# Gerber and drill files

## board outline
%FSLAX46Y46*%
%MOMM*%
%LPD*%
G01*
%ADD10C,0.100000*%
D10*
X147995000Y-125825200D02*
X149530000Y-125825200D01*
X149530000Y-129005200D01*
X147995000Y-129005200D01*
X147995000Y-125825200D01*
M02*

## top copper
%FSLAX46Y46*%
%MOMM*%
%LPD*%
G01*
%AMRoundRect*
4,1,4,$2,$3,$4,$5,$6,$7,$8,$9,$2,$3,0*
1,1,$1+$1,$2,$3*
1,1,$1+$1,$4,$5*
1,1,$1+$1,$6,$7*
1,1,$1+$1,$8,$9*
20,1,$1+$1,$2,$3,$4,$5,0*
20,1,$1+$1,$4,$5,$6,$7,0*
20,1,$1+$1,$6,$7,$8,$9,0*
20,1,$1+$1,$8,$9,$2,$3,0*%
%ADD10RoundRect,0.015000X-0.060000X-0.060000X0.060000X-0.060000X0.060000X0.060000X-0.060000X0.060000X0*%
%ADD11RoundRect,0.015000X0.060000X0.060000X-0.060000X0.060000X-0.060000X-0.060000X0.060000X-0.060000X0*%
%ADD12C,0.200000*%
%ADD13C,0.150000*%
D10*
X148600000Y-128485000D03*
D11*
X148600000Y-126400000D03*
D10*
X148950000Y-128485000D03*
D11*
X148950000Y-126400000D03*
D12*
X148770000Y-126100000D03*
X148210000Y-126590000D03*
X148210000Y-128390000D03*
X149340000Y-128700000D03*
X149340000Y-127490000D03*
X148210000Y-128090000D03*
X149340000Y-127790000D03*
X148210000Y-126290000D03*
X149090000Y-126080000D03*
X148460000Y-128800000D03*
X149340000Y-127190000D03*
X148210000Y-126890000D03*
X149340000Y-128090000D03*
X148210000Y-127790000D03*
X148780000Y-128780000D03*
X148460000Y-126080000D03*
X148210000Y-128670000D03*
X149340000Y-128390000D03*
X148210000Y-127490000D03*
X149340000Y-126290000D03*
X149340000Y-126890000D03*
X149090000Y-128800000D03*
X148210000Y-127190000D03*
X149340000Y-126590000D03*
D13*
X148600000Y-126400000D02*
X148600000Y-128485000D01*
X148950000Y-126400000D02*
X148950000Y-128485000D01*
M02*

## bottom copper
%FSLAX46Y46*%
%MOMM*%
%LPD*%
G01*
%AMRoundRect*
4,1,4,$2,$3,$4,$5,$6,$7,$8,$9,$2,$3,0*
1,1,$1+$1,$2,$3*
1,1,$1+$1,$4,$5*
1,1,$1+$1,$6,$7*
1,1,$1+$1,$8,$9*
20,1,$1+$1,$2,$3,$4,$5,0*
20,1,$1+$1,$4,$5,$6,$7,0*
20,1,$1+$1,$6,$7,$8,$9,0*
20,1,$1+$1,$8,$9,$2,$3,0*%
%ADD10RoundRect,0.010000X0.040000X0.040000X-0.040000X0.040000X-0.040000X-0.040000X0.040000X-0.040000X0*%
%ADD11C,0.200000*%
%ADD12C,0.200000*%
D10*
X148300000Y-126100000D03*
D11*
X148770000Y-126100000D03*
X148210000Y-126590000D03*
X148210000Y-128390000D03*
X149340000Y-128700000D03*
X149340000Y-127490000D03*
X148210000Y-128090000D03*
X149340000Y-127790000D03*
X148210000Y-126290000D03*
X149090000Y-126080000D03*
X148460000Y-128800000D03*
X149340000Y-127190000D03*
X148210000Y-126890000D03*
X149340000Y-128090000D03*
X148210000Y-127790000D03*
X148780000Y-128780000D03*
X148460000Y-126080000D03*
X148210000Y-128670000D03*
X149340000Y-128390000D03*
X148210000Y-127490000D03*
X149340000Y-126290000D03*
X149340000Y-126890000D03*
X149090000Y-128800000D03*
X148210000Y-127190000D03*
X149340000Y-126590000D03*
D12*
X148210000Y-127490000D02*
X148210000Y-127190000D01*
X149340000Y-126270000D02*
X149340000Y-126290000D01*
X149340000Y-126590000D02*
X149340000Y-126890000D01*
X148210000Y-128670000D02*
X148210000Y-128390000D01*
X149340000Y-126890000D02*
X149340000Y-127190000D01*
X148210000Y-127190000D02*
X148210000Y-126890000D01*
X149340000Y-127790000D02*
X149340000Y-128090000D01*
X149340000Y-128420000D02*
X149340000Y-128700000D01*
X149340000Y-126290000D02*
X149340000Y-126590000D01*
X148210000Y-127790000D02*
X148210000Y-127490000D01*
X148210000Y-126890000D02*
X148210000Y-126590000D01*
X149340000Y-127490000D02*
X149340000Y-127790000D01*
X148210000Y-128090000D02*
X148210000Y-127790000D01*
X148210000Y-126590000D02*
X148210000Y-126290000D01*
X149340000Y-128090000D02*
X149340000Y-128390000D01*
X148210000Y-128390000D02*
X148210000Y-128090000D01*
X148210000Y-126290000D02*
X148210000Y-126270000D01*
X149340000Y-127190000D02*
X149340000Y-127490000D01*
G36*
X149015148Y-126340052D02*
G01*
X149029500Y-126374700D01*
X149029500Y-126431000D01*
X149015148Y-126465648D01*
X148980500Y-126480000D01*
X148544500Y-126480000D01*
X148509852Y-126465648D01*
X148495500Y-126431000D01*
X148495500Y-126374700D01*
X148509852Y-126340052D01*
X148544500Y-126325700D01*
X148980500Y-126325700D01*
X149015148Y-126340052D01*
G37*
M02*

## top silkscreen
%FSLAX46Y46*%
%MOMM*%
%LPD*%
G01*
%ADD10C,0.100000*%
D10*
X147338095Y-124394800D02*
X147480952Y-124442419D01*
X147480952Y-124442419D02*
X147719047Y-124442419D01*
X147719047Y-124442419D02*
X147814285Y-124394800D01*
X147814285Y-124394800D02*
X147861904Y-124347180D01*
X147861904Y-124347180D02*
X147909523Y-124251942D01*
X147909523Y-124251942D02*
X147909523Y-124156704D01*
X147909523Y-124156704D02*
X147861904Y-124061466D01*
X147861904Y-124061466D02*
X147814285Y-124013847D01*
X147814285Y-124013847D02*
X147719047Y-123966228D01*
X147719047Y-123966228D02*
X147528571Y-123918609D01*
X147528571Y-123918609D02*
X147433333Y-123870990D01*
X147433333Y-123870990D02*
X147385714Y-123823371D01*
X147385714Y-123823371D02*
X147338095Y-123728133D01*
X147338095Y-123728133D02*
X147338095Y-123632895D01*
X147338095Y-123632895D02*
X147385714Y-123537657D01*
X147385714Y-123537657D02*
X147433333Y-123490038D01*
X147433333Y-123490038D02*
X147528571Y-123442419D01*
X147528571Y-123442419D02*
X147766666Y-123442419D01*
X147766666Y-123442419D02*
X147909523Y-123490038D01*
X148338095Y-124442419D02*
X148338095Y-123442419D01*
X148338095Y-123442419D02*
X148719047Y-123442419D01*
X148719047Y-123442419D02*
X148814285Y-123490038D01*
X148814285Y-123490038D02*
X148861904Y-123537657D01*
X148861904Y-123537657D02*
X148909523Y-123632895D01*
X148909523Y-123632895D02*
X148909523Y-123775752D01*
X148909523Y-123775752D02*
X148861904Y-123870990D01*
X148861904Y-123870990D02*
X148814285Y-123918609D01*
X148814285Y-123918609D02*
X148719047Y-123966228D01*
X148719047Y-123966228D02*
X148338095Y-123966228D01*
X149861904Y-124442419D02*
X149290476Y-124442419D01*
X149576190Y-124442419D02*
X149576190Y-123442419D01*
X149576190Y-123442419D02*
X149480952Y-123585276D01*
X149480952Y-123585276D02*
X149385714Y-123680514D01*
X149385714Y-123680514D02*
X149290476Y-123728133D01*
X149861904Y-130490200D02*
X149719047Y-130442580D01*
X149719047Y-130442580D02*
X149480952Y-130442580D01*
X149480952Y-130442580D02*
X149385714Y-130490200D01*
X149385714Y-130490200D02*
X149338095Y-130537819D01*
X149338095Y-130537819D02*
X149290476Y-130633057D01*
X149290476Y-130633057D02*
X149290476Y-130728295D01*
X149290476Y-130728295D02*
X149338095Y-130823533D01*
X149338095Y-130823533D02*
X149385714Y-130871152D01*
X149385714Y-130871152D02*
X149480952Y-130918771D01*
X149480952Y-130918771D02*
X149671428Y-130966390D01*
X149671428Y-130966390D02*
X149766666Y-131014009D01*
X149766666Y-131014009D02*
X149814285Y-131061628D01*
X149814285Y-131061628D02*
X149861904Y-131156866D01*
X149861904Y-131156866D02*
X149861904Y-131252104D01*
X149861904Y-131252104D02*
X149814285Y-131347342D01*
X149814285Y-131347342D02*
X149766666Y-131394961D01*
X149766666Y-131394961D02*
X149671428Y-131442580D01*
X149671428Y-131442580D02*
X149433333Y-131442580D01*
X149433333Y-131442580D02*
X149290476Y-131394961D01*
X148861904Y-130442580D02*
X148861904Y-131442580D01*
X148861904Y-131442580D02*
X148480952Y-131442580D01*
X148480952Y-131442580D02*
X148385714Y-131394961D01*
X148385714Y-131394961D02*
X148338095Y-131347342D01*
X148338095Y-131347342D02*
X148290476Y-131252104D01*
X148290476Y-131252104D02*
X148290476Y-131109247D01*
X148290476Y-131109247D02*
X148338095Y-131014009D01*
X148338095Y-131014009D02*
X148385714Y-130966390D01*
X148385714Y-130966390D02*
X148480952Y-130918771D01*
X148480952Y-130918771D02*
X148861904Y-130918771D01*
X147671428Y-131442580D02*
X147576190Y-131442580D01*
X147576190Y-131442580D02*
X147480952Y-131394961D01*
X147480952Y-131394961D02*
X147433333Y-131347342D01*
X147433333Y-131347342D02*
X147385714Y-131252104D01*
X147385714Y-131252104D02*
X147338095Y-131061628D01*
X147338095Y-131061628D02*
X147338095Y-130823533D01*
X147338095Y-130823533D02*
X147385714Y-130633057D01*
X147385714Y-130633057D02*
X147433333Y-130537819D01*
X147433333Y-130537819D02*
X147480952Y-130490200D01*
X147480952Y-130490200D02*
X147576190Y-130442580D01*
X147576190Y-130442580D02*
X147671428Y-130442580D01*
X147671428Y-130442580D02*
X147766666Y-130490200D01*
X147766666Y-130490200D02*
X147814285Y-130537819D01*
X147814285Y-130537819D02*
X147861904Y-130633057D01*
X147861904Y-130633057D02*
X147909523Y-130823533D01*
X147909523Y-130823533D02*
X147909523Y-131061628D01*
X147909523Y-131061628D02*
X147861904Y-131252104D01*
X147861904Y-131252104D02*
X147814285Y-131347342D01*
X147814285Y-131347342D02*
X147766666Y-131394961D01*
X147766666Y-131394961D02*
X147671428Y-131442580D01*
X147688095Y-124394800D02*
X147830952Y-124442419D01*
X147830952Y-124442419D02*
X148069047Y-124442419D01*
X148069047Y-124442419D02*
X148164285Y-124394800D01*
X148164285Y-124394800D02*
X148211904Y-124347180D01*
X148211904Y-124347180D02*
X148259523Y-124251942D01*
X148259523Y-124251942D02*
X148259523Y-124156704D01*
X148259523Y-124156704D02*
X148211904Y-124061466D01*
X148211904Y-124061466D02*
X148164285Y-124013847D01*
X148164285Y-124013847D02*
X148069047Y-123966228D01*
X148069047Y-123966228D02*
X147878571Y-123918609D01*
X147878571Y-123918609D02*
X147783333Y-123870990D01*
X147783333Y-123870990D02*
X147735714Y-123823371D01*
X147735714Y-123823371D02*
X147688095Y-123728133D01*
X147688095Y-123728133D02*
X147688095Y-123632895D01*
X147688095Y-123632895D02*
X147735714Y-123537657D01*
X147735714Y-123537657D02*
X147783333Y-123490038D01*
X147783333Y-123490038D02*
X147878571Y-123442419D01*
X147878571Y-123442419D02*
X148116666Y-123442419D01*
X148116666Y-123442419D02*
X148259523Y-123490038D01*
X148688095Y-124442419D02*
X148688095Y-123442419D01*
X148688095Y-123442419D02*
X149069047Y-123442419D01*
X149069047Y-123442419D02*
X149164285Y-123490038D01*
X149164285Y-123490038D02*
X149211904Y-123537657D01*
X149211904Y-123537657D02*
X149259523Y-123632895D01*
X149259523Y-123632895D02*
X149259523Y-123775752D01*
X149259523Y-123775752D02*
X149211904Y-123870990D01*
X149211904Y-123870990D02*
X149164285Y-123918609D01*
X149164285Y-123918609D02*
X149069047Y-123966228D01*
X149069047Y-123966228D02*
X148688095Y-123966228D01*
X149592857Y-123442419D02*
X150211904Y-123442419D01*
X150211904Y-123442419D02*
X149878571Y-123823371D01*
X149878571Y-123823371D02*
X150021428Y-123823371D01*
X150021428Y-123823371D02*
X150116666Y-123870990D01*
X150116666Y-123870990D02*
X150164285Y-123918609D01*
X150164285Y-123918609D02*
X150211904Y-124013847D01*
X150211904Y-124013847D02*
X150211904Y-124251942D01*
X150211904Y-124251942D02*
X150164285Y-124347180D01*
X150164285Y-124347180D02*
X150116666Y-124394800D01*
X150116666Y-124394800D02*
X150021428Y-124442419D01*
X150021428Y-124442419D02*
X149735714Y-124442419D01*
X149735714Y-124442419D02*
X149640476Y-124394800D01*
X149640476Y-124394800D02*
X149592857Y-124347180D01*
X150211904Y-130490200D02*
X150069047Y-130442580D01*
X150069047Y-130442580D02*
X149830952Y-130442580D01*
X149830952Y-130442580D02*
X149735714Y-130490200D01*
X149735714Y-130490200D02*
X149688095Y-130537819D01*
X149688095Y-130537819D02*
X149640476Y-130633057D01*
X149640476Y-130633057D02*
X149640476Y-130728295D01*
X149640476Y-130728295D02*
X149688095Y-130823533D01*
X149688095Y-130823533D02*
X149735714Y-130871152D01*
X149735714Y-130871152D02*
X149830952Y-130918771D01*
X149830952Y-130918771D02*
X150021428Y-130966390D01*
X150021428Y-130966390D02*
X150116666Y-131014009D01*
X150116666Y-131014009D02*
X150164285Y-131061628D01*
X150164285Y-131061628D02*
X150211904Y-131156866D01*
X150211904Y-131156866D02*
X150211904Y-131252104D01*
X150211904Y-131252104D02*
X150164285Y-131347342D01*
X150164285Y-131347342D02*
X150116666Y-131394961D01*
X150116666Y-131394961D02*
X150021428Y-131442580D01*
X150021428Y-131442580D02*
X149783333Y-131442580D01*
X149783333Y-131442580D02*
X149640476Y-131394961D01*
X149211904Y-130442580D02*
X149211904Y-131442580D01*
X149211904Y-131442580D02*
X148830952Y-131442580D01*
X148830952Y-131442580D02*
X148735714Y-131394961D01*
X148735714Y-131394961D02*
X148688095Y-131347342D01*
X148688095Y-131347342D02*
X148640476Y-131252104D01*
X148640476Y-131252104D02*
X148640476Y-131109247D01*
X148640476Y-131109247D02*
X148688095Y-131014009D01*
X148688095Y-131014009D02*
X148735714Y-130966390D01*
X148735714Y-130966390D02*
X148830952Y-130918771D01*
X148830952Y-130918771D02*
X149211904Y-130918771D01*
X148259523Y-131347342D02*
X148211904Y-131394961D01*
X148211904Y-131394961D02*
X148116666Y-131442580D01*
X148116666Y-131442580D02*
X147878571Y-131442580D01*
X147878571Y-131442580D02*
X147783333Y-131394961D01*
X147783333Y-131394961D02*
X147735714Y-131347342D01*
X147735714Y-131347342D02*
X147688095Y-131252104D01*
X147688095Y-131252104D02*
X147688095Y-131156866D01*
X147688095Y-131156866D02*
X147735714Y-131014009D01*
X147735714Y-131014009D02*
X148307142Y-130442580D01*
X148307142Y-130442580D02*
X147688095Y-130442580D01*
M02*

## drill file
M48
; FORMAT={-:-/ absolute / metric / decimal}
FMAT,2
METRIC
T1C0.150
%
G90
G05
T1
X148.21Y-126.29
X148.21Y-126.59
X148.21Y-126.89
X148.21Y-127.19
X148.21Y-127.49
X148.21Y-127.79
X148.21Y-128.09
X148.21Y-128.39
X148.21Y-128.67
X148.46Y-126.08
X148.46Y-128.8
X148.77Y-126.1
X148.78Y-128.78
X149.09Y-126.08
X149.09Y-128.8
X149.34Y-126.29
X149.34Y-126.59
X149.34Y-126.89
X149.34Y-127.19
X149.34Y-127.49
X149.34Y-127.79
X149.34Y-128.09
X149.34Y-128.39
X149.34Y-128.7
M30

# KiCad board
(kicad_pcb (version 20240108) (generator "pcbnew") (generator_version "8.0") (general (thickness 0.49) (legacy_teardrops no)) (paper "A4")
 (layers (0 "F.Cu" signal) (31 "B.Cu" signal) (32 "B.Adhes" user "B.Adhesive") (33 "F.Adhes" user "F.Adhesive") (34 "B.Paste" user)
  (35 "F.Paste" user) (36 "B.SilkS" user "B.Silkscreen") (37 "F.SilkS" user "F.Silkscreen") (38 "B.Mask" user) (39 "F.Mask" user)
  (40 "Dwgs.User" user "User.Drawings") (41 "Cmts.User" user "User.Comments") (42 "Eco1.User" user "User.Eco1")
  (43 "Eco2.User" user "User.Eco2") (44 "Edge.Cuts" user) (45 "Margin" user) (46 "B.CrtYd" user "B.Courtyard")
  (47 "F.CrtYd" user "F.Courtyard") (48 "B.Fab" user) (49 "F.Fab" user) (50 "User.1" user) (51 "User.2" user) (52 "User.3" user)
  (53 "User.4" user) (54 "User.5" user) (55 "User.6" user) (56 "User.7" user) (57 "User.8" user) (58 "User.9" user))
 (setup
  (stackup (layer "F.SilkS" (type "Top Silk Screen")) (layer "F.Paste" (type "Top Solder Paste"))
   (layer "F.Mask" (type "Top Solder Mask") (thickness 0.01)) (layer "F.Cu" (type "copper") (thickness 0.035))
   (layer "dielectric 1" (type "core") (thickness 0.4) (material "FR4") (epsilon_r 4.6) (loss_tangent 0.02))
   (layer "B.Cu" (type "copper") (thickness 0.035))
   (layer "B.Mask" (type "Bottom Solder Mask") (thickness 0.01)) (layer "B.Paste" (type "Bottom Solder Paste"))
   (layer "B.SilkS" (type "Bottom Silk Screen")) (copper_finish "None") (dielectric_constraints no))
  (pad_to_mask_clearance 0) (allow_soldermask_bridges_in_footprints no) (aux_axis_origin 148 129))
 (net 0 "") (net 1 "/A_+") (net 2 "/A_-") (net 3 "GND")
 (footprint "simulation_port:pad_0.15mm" (layer "F.Cu") (at 148.6 128.485)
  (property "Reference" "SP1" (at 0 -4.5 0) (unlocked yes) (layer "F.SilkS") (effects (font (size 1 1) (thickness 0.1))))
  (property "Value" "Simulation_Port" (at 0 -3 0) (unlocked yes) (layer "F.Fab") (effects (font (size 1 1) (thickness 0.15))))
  (pad "1" smd roundrect (at 0 0) (size 0.15 0.15) (layers "F.Cu" "F.Paste" "F.Mask") (roundrect_rratio 0.1) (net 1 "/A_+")
   (thermal_bridge_angle 45)
   (teardrops (best_length_ratio 0.5) (max_length 1) (best_width_ratio 1) (max_width 2) (curve_points 0) (filter_ratio 0.9) (enabled yes)
    (allow_two_segments yes) (prefer_zone_connections yes))))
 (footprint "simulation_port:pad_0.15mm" (layer "F.Cu") (at 148.6 126.4 180)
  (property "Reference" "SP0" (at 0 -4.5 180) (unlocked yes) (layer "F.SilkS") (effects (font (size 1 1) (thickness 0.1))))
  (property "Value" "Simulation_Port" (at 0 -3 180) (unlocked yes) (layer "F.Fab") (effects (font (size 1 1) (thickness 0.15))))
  (pad "1" smd roundrect (at 0 0 180) (size 0.15 0.15) (layers "F.Cu" "F.Paste" "F.Mask") (roundrect_rratio 0.1) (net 1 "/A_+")
   (thermal_bridge_angle 45)
   (teardrops (best_length_ratio 0.5) (max_length 1) (best_width_ratio 1) (max_width 2) (curve_points 0) (filter_ratio 0.9) (enabled yes)
    (allow_two_segments yes) (prefer_zone_connections yes))))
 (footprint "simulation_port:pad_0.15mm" (layer "F.Cu") (at 148.95 128.485)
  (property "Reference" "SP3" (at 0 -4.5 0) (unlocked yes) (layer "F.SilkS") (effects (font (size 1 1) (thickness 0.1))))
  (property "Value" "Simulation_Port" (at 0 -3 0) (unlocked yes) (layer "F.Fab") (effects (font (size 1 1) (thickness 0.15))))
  (pad "1" smd roundrect (at 0 0) (size 0.15 0.15) (layers "F.Cu" "F.Paste" "F.Mask") (roundrect_rratio 0.1) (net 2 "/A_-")
   (thermal_bridge_angle 45)
   (teardrops (best_length_ratio 0.5) (max_length 1) (best_width_ratio 1) (max_width 2) (curve_points 0) (filter_ratio 0.9) (enabled yes)
    (allow_two_segments yes) (prefer_zone_connections yes))))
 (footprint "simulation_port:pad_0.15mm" (layer "F.Cu") (at 148.95 126.4 180)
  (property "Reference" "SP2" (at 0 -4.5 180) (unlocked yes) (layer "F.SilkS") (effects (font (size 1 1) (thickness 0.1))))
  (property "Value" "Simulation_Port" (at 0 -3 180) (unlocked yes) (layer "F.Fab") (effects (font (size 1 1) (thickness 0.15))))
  (pad "1" smd roundrect (at 0 0 180) (size 0.15 0.15) (layers "F.Cu" "F.Paste" "F.Mask") (roundrect_rratio 0.1) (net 2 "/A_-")
   (thermal_bridge_angle 45)
   (teardrops (best_length_ratio 0.5) (max_length 1) (best_width_ratio 1) (max_width 2) (curve_points 0) (filter_ratio 0.9) (enabled yes)
    (allow_two_segments yes) (prefer_zone_connections yes))))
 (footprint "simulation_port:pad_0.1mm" (layer "B.Cu") (at 148.3 126.1 180)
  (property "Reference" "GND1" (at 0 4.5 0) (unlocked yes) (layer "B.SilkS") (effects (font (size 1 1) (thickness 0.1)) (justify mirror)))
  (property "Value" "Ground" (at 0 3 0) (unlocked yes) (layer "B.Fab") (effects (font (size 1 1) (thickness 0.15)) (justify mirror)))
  (pad "1" smd roundrect (at 0 0 180) (size 0.1 0.1) (layers "B.Cu" "B.Paste" "B.Mask") (roundrect_rratio 0.1) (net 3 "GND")
   (thermal_bridge_angle 45)
   (teardrops (best_length_ratio 0.5) (max_length 1) (best_width_ratio 1) (max_width 2) (curve_points 0) (filter_ratio 0.9) (enabled yes)
    (allow_two_segments yes) (prefer_zone_connections yes))))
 (gr_rect (start 147.995 125.8252) (end 149.53 129.0052) (stroke (width 0.1) (type solid)) (fill none) (layer "Edge.Cuts"))
 (via (at 148.77 126.1) (size 0.2) (drill 0.15) (layers "F.Cu" "B.Cu") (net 3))
 (via (at 148.21 126.59) (size 0.2) (drill 0.15) (layers "F.Cu" "B.Cu") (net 3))
 (via (at 148.21 128.39) (size 0.2) (drill 0.15) (layers "F.Cu" "B.Cu") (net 3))
 (via (at 149.34 128.7) (size 0.2) (drill 0.15) (layers "F.Cu" "B.Cu") (free yes) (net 3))
 (via (at 149.34 127.49) (size 0.2) (drill 0.15) (layers "F.Cu" "B.Cu") (free yes) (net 3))
 (via (at 148.21 128.09) (size 0.2) (drill 0.15) (layers "F.Cu" "B.Cu")
  (teardrops (best_length_ratio 0.5) (max_length 1) (best_width_ratio 1) (max_width 2) (curve_points 0) (filter_ratio 0.9) (enabled no)
   (allow_two_segments no) (prefer_zone_connections yes))
  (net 3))
 (via (at 149.34 127.79) (size 0.2) (drill 0.15) (layers "F.Cu" "B.Cu") (free yes) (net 3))
 (via (at 148.21 126.29) (size 0.2) (drill 0.15) (layers "F.Cu" "B.Cu") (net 3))
 (via (at 149.09 126.08) (size 0.2) (drill 0.15) (layers "F.Cu" "B.Cu") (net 3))
 (via (at 148.46 128.8) (size 0.2) (drill 0.15) (layers "F.Cu" "B.Cu") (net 3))
 (via (at 149.34 127.19) (size 0.2) (drill 0.15) (layers "F.Cu" "B.Cu") (free yes) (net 3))
 (via (at 148.21 126.89) (size 0.2) (drill 0.15) (layers "F.Cu" "B.Cu") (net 3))
 (via (at 149.34 128.09) (size 0.2) (drill 0.15) (layers "F.Cu" "B.Cu") (free yes) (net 3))
 (via (at 148.21 127.79) (size 0.2) (drill 0.15) (layers "F.Cu" "B.Cu") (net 3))
 (via (at 148.78 128.78) (size 0.2) (drill 0.15) (layers "F.Cu" "B.Cu") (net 3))
 (via (at 148.46 126.08) (size 0.2) (drill 0.15) (layers "F.Cu" "B.Cu") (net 3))
 (via (at 148.21 128.67) (size 0.2) (drill 0.15) (layers "F.Cu" "B.Cu") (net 3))
 (via (at 149.34 128.39) (size 0.2) (drill 0.15) (layers "F.Cu" "B.Cu") (free yes) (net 3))
 (via (at 148.21 127.49) (size 0.2) (drill 0.15) (layers "F.Cu" "B.Cu") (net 3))
 (via (at 149.34 126.29) (size 0.2) (drill 0.15) (layers "F.Cu" "B.Cu") (free yes) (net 3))
 (via (at 149.34 126.89) (size 0.2) (drill 0.15) (layers "F.Cu" "B.Cu") (free yes) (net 3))
 (via (at 149.09 128.8) (size 0.2) (drill 0.15) (layers "F.Cu" "B.Cu") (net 3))
 (via (at 148.21 127.19) (size 0.2) (drill 0.15) (layers "F.Cu" "B.Cu") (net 3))
 (via (at 149.34 126.59) (size 0.2) (drill 0.15) (layers "F.Cu" "B.Cu") (free yes) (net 3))
 (segment (start 148.21 127.49) (end 148.21 127.19) (width 0.2) (layer "B.Cu") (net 3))
 (segment (start 149.34 126.27) (end 149.34 126.29) (width 0.2) (layer "B.Cu") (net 3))
 (segment (start 149.34 126.59) (end 149.34 126.89) (width 0.2) (layer "B.Cu") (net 3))
 (segment (start 148.21 128.67) (end 148.21 128.39) (width 0.2) (layer "B.Cu") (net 3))
 (segment (start 149.34 126.89) (end 149.34 127.19) (width 0.2) (layer "B.Cu") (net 3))
 (segment (start 148.21 127.19) (end 148.21 126.89) (width 0.2) (layer "B.Cu") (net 3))
 (segment (start 149.34 127.79) (end 149.34 128.09) (width 0.2) (layer "B.Cu") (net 3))
 (segment (start 149.34 128.42) (end 149.34 128.7) (width 0.2) (layer "B.Cu") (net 3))
 (segment (start 149.34 126.29) (end 149.34 126.59) (width 0.2) (layer "B.Cu") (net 3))
 (segment (start 148.21 127.79) (end 148.21 127.49) (width 0.2) (layer "B.Cu") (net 3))
 (segment (start 148.21 126.89) (end 148.21 126.59) (width 0.2) (layer "B.Cu") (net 3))
 (segment (start 149.34 127.49) (end 149.34 127.79) (width 0.2) (layer "B.Cu") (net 3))
 (segment (start 148.21 128.09) (end 148.21 127.79) (width 0.2) (layer "B.Cu") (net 3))
 (segment (start 148.21 126.59) (end 148.21 126.29) (width 0.2) (layer "B.Cu") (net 3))
 (segment (start 149.34 128.09) (end 149.34 128.39) (width 0.2) (layer "B.Cu") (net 3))
 (segment (start 148.21 128.39) (end 148.21 128.09) (width 0.2) (layer "B.Cu") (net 3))
 (segment (start 148.21 126.29) (end 148.21 126.27) (width 0.2) (layer "B.Cu") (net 3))
 (segment (start 149.34 127.19) (end 149.34 127.49) (width 0.2) (layer "B.Cu") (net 3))
 (segment (start 148.6 126.4) (end 148.6 128.485) (width 0.15) (layer "F.Cu") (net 1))
 (segment (start 148.95 126.4) (end 148.95 128.485) (width 0.15) (layer "F.Cu") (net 2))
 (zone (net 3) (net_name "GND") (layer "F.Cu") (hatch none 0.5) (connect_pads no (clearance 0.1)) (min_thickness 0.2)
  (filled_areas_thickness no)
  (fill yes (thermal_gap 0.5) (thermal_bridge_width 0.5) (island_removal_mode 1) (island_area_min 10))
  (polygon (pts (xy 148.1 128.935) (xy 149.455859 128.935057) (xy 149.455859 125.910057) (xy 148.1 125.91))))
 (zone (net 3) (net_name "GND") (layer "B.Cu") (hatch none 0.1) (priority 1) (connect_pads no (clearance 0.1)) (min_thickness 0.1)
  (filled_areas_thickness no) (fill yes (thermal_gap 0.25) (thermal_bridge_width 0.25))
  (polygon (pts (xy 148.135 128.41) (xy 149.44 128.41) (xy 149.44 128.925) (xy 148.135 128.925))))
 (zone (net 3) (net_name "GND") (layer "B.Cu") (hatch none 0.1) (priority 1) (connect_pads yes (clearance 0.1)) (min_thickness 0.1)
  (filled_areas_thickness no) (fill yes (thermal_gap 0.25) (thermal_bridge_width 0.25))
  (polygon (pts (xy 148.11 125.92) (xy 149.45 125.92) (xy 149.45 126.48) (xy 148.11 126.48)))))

